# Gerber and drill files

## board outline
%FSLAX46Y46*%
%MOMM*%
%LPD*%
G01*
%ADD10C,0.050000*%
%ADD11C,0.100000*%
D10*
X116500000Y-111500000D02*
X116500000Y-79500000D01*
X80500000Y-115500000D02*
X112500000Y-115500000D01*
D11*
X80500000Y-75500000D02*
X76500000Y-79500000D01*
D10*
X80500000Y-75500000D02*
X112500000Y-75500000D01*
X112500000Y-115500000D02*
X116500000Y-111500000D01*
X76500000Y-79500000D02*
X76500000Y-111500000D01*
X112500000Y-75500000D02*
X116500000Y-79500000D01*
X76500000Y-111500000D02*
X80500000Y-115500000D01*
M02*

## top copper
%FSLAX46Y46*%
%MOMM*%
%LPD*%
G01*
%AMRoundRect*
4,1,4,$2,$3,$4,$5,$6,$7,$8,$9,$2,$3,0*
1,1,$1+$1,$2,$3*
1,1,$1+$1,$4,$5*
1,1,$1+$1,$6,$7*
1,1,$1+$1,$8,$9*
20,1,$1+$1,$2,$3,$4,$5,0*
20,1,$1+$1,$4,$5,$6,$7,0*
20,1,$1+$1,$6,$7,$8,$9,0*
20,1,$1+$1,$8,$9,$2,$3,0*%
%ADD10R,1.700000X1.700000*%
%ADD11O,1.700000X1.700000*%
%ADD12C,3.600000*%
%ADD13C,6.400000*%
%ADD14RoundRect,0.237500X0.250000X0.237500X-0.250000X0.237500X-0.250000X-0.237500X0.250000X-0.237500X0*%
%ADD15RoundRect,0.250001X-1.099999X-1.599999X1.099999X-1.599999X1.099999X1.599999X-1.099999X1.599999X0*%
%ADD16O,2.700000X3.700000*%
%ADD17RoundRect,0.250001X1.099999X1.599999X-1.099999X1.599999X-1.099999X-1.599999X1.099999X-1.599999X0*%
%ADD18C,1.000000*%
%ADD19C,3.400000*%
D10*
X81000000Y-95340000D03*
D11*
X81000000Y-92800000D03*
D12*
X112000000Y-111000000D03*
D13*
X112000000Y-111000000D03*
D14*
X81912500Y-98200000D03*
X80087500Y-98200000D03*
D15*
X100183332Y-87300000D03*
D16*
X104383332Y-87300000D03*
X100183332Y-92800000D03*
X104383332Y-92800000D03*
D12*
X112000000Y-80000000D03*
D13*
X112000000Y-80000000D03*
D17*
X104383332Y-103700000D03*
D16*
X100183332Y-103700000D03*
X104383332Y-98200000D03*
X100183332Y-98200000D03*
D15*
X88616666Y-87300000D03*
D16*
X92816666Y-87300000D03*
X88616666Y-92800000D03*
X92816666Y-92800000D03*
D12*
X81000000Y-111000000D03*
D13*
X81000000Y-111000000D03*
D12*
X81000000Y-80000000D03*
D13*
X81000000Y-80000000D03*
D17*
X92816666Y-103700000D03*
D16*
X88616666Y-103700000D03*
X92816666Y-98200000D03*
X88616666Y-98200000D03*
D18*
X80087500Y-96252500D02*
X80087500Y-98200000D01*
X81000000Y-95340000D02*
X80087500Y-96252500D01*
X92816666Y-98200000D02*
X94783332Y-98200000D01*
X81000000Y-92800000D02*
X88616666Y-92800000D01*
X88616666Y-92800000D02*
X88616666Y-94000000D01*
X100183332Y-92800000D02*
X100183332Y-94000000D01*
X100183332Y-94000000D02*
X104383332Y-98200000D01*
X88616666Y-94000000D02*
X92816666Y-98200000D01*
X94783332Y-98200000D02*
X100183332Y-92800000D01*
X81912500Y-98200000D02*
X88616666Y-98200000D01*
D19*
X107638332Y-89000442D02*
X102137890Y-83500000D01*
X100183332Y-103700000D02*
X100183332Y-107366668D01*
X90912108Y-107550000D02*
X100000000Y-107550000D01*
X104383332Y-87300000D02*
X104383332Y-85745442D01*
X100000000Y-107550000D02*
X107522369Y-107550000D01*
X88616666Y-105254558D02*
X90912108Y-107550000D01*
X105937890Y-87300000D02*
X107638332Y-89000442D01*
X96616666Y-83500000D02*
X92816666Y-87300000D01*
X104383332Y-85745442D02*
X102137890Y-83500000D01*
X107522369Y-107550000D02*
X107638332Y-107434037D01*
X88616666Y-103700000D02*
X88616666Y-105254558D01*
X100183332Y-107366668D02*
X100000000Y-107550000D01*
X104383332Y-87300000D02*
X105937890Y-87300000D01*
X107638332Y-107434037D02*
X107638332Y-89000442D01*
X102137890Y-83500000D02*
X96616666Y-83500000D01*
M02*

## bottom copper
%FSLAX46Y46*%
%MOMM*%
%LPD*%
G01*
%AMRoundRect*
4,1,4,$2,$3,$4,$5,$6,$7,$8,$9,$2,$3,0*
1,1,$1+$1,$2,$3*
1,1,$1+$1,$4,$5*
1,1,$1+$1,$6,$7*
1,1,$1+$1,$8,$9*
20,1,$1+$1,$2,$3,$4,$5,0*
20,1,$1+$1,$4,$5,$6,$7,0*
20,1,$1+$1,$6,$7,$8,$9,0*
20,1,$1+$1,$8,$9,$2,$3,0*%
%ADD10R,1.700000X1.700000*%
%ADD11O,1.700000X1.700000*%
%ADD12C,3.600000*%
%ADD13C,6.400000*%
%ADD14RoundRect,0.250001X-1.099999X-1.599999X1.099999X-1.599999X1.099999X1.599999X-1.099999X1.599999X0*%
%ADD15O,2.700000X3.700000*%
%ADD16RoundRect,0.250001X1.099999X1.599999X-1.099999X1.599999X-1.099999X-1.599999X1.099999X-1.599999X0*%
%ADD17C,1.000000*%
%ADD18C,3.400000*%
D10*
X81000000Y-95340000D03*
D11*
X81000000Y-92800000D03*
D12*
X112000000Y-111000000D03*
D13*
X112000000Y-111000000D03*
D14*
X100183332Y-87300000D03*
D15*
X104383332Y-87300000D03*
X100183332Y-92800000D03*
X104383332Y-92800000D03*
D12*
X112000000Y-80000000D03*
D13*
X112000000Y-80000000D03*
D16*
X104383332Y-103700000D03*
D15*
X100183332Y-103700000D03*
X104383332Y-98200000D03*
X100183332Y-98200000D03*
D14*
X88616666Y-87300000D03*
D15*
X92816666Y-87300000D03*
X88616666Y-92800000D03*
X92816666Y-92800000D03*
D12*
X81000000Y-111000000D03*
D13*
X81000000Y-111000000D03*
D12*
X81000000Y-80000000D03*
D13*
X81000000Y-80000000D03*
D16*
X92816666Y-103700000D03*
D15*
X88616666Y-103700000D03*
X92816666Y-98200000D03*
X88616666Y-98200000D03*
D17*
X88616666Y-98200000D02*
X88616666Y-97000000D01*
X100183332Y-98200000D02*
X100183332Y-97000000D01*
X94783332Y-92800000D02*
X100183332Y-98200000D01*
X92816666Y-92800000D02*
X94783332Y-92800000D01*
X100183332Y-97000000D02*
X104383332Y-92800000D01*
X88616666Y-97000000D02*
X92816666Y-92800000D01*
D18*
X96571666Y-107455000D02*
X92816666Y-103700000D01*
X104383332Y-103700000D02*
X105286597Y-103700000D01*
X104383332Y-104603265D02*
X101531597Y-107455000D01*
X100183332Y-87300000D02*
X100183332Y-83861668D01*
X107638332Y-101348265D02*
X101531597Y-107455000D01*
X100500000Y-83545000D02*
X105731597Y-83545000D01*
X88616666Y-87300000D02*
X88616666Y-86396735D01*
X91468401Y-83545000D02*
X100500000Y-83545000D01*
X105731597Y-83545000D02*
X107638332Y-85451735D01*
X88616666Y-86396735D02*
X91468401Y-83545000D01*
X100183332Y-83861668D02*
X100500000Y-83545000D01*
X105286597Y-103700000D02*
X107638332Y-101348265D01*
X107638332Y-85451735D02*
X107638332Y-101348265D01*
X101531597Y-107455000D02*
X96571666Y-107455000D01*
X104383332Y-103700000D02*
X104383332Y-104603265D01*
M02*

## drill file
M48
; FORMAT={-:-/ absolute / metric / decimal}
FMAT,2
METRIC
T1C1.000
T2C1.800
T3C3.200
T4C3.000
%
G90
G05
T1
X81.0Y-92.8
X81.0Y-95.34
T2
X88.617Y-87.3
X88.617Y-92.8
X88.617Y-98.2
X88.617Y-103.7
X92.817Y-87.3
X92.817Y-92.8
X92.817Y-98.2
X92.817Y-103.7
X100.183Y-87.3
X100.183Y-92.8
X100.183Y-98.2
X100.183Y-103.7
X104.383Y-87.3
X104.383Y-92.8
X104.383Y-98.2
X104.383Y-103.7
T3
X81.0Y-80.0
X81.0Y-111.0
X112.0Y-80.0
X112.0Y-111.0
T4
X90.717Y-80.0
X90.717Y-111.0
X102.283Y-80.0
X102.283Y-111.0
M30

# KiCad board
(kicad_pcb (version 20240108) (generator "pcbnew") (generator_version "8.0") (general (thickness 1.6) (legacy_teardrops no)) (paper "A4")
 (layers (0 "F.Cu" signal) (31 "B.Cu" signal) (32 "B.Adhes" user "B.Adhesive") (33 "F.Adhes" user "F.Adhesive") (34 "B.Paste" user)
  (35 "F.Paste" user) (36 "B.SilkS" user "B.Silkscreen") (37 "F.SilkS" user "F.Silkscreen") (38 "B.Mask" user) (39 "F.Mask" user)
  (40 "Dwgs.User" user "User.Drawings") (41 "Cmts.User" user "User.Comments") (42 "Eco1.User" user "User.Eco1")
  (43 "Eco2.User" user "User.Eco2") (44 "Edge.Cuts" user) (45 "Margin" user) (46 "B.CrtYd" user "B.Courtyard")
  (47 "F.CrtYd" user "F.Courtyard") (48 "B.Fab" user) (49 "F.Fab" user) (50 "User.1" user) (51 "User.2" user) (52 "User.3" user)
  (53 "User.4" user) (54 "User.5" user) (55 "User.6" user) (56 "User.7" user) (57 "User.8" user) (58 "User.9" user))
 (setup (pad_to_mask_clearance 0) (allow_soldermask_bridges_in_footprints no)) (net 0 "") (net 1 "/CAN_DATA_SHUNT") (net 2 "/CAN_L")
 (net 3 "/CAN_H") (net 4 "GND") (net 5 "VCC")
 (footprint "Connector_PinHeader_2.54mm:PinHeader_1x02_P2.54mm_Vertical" (layer "F.Cu") (at 81 95.34 180)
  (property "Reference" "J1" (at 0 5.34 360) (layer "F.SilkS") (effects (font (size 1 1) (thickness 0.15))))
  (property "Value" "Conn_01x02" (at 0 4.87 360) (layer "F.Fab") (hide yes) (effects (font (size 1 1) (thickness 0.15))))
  (pad "1" thru_hole rect (at 0 0 180) (size 1.7 1.7) (drill 1) (layers "*.Cu" "*.Mask") (remove_unused_layers no) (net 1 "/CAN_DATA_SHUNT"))
  (pad "2" thru_hole oval (at 0 2.54 180) (size 1.7 1.7) (drill 1) (layers "*.Cu" "*.Mask") (remove_unused_layers no) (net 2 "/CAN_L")))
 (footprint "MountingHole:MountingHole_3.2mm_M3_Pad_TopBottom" (layer "F.Cu") (at 112 111)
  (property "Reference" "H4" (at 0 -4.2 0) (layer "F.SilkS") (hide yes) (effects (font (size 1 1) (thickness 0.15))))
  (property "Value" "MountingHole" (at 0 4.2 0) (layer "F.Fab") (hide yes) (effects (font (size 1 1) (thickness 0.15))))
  (pad "1" thru_hole circle (at 0 0) (size 3.6 3.6) (drill 3.2) (layers "*.Cu" "*.Mask") (remove_unused_layers no))
  (pad "1" connect circle (at 0 0) (size 6.4 6.4) (layers "F.Cu" "F.Mask"))
  (pad "1" connect circle (at 0 0) (size 6.4 6.4) (layers "B.Cu" "B.Mask")))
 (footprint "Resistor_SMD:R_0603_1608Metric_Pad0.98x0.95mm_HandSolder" (layer "F.Cu") (at 81 98.2 180)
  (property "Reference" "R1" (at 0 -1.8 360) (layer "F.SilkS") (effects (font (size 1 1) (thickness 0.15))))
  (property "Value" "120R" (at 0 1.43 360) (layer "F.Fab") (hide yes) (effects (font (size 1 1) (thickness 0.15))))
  (pad "1" smd roundrect (at -0.9125 0 180) (size 0.975 0.95) (layers "F.Cu" "F.Paste" "F.Mask") (roundrect_rratio 0.25) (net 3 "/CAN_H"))
  (pad "2" smd roundrect (at 0.9125 0 180) (size 0.975 0.95) (layers "F.Cu" "F.Paste" "F.Mask") (roundrect_rratio 0.25)
   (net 1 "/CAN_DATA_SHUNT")))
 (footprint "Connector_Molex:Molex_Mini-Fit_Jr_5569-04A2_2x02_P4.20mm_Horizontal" (layer "F.Cu") (at 100.183332 87.3)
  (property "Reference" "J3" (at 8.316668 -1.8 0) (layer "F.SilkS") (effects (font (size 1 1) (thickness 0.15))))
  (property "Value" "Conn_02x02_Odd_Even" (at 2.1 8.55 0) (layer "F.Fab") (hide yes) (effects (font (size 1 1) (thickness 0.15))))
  (pad "" np_thru_hole circle (at 2.1 -7.3) (size 3 3) (drill 3) (layers "*.Cu" "*.Mask"))
  (pad "1" thru_hole roundrect (at 0 0) (size 2.7 3.7) (drill 1.8) (layers "*.Cu" "*.Mask") (remove_unused_layers no)
   (roundrect_rratio 0.092593) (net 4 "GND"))
  (pad "2" thru_hole oval (at 4.2 0) (size 2.7 3.7) (drill 1.8) (layers "*.Cu" "*.Mask") (remove_unused_layers no) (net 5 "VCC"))
  (pad "3" thru_hole oval (at 0 5.5) (size 2.7 3.7) (drill 1.8) (layers "*.Cu" "*.Mask") (remove_unused_layers no) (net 2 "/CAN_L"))
  (pad "4" thru_hole oval (at 4.2 5.5) (size 2.7 3.7) (drill 1.8) (layers "*.Cu" "*.Mask") (remove_unused_layers no) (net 3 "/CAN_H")))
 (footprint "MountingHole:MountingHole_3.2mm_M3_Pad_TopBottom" (layer "F.Cu") (at 112 80)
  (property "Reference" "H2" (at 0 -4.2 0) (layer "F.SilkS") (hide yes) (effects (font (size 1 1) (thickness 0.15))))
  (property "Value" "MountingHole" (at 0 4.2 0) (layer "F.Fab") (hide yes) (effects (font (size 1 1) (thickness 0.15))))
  (pad "1" thru_hole circle (at 0 0) (size 3.6 3.6) (drill 3.2) (layers "*.Cu" "*.Mask") (remove_unused_layers no))
  (pad "1" connect circle (at 0 0) (size 6.4 6.4) (layers "F.Cu" "F.Mask"))
  (pad "1" connect circle (at 0 0) (size 6.4 6.4) (layers "B.Cu" "B.Mask")))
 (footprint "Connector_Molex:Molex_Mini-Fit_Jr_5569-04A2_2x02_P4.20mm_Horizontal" (layer "F.Cu") (at 104.383332 103.7 180)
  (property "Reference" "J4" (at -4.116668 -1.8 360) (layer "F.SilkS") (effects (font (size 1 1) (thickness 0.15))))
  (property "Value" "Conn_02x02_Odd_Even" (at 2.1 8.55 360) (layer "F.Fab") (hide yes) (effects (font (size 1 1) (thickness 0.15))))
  (pad "" np_thru_hole circle (at 2.1 -7.3 180) (size 3 3) (drill 3) (layers "*.Cu" "*.Mask"))
  (pad "1" thru_hole roundrect (at 0 0 180) (size 2.7 3.7) (drill 1.8) (layers "*.Cu" "*.Mask") (remove_unused_layers no)
   (roundrect_rratio 0.092593) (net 4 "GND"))
  (pad "2" thru_hole oval (at 4.2 0 180) (size 2.7 3.7) (drill 1.8) (layers "*.Cu" "*.Mask") (remove_unused_layers no) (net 5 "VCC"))
  (pad "3" thru_hole oval (at 0 5.5 180) (size 2.7 3.7) (drill 1.8) (layers "*.Cu" "*.Mask") (remove_unused_layers no) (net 2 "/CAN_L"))
  (pad "4" thru_hole oval (at 4.2 5.5 180) (size 2.7 3.7) (drill 1.8) (layers "*.Cu" "*.Mask") (remove_unused_layers no) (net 3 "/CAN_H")))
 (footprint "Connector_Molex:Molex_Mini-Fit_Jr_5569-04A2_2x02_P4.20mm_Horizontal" (layer "F.Cu") (at 88.616666 87.3)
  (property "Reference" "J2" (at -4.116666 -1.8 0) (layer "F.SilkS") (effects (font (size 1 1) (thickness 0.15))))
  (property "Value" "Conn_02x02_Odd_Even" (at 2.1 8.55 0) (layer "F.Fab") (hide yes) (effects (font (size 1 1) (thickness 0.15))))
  (pad "" np_thru_hole circle (at 2.1 -7.3) (size 3 3) (drill 3) (layers "*.Cu" "*.Mask"))
  (pad "1" thru_hole roundrect (at 0 0) (size 2.7 3.7) (drill 1.8) (layers "*.Cu" "*.Mask") (remove_unused_layers no)
   (roundrect_rratio 0.092593) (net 4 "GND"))
  (pad "2" thru_hole oval (at 4.2 0) (size 2.7 3.7) (drill 1.8) (layers "*.Cu" "*.Mask") (remove_unused_layers no) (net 5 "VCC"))
  (pad "3" thru_hole oval (at 0 5.5) (size 2.7 3.7) (drill 1.8) (layers "*.Cu" "*.Mask") (remove_unused_layers no) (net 2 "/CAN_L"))
  (pad "4" thru_hole oval (at 4.2 5.5) (size 2.7 3.7) (drill 1.8) (layers "*.Cu" "*.Mask") (remove_unused_layers no) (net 3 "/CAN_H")))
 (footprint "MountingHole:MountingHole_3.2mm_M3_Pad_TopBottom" (layer "F.Cu") (at 81 111)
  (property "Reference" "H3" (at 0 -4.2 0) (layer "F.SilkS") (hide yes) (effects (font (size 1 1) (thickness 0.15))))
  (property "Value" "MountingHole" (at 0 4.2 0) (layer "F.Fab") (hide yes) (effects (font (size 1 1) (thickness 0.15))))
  (pad "1" thru_hole circle (at 0 0) (size 3.6 3.6) (drill 3.2) (layers "*.Cu" "*.Mask") (remove_unused_layers no))
  (pad "1" connect circle (at 0 0) (size 6.4 6.4) (layers "F.Cu" "F.Mask"))
  (pad "1" connect circle (at 0 0) (size 6.4 6.4) (layers "B.Cu" "B.Mask")))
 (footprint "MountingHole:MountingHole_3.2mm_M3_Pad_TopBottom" (layer "F.Cu") (at 81 80)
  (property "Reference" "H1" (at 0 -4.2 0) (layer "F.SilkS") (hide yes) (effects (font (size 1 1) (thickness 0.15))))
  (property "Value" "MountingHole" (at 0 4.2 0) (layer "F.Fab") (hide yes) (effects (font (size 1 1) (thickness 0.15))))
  (pad "1" thru_hole circle (at 0 0) (size 3.6 3.6) (drill 3.2) (layers "*.Cu" "*.Mask") (remove_unused_layers no))
  (pad "1" connect circle (at 0 0) (size 6.4 6.4) (layers "F.Cu" "F.Mask"))
  (pad "1" connect circle (at 0 0) (size 6.4 6.4) (layers "B.Cu" "B.Mask")))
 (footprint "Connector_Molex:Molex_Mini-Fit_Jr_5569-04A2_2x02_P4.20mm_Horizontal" (layer "F.Cu") (at 92.816666 103.7 180)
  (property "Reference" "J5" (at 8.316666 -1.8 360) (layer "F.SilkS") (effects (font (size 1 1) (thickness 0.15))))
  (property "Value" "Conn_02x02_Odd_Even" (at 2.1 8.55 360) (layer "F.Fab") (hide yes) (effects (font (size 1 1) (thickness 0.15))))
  (pad "" np_thru_hole circle (at 2.1 -7.3 180) (size 3 3) (drill 3) (layers "*.Cu" "*.Mask"))
  (pad "1" thru_hole roundrect (at 0 0 180) (size 2.7 3.7) (drill 1.8) (layers "*.Cu" "*.Mask") (remove_unused_layers no)
   (roundrect_rratio 0.092593) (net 4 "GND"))
  (pad "2" thru_hole oval (at 4.2 0 180) (size 2.7 3.7) (drill 1.8) (layers "*.Cu" "*.Mask") (remove_unused_layers no) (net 5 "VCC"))
  (pad "3" thru_hole oval (at 0 5.5 180) (size 2.7 3.7) (drill 1.8) (layers "*.Cu" "*.Mask") (remove_unused_layers no) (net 2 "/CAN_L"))
  (pad "4" thru_hole oval (at 4.2 5.5 180) (size 2.7 3.7) (drill 1.8) (layers "*.Cu" "*.Mask") (remove_unused_layers no) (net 3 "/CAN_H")))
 (gr_line (start 116.5 111.5) (end 116.5 79.5) (stroke (width 0.05) (type default)) (layer "Edge.Cuts"))
 (gr_line (start 80.5 115.5) (end 112.5 115.5) (stroke (width 0.05) (type default)) (layer "Edge.Cuts"))
 (gr_line (start 80.5 75.5) (end 76.5 79.5) (stroke (width 0.1) (type default)) (layer "Edge.Cuts"))
 (gr_line (start 80.5 75.5) (end 112.5 75.5) (stroke (width 0.05) (type default)) (layer "Edge.Cuts"))
 (gr_line (start 112.5 115.5) (end 116.5 111.5) (stroke (width 0.05) (type default)) (layer "Edge.Cuts"))
 (gr_line (start 76.5 79.5) (end 76.5 111.5) (stroke (width 0.05) (type default)) (layer "Edge.Cuts"))
 (gr_line (start 112.5 75.5) (end 116.5 79.5) (stroke (width 0.05) (type default)) (layer "Edge.Cuts"))
 (gr_line (start 76.5 111.5) (end 80.5 115.5) (stroke (width 0.05) (type default)) (layer "Edge.Cuts"))
 (segment (start 80.0875 96.2525) (end 80.0875 98.2) (width 1) (layer "F.Cu") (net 1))
 (segment (start 81 95.34) (end 80.0875 96.2525) (width 1) (layer "F.Cu") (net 1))
 (segment (start 92.816666 98.2) (end 94.783332 98.2) (width 1) (layer "F.Cu") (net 2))
 (segment (start 81 92.8) (end 88.616666 92.8) (width 1) (layer "F.Cu") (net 2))
 (segment (start 88.616666 92.8) (end 88.616666 94) (width 1) (layer "F.Cu") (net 2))
 (segment (start 100.183332 92.8) (end 100.183332 94) (width 1) (layer "F.Cu") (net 2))
 (segment (start 100.183332 94) (end 104.383332 98.2) (width 1) (layer "F.Cu") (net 2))
 (segment (start 88.616666 94) (end 92.816666 98.2) (width 1) (layer "F.Cu") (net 2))
 (segment (start 94.783332 98.2) (end 100.183332 92.8) (width 1) (layer "F.Cu") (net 2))
 (segment (start 81.9125 98.2) (end 88.616666 98.2) (width 1) (layer "F.Cu") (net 3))
 (segment (start 88.616666 98.2) (end 88.616666 97) (width 1) (layer "B.Cu") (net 3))
 (segment (start 100.183332 98.2) (end 100.183332 97) (width 1) (layer "B.Cu") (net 3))
 (segment (start 94.783332 92.8) (end 100.183332 98.2) (width 1) (layer "B.Cu") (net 3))
 (segment (start 92.816666 92.8) (end 94.783332 92.8) (width 1) (layer "B.Cu") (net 3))
 (segment (start 100.183332 97) (end 104.383332 92.8) (width 1) (layer "B.Cu") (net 3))
 (segment (start 88.616666 97) (end 92.816666 92.8) (width 1) (layer "B.Cu") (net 3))
 (segment (start 96.571666 107.455) (end 92.816666 103.7) (width 3.4) (layer "B.Cu") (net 4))
 (segment (start 104.383332 103.7) (end 105.286597 103.7) (width 3.4) (layer "B.Cu") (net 4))
 (segment (start 104.383332 104.603265) (end 101.531597 107.455) (width 3.4) (layer "B.Cu") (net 4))
 (segment (start 100.183332 87.3) (end 100.183332 83.861668) (width 3.4) (layer "B.Cu") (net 4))
 (segment (start 107.638332 101.348265) (end 101.531597 107.455) (width 3.4) (layer "B.Cu") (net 4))
 (segment (start 100.5 83.545) (end 105.731597 83.545) (width 3.4) (layer "B.Cu") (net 4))
 (segment (start 88.616666 87.3) (end 88.616666 86.396735) (width 3.4) (layer "B.Cu") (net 4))
 (segment (start 91.468401 83.545) (end 100.5 83.545) (width 3.4) (layer "B.Cu") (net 4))
 (segment (start 105.731597 83.545) (end 107.638332 85.451735) (width 3.4) (layer "B.Cu") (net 4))
 (segment (start 88.616666 86.396735) (end 91.468401 83.545) (width 3.4) (layer "B.Cu") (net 4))
 (segment (start 100.183332 83.861668) (end 100.5 83.545) (width 3.4) (layer "B.Cu") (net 4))
 (segment (start 105.286597 103.7) (end 107.638332 101.348265) (width 3.4) (layer "B.Cu") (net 4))
 (segment (start 107.638332 85.451735) (end 107.638332 101.348265) (width 3.4) (layer "B.Cu") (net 4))
 (segment (start 101.531597 107.455) (end 96.571666 107.455) (width 3.4) (layer "B.Cu") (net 4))
 (segment (start 104.383332 103.7) (end 104.383332 104.603265) (width 3.4) (layer "B.Cu") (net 4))
 (segment (start 107.638332 89.000442) (end 102.13789 83.5) (width 3.4) (layer "F.Cu") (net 5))
 (segment (start 100.183332 103.7) (end 100.183332 107.366668) (width 3.4) (layer "F.Cu") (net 5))
 (segment (start 90.912108 107.55) (end 100 107.55) (width 3.4) (layer "F.Cu") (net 5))
 (segment (start 104.383332 87.3) (end 104.383332 85.745442) (width 3.4) (layer "F.Cu") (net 5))
 (segment (start 100 107.55) (end 107.522369 107.55) (width 3.4) (layer "F.Cu") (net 5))
 (segment (start 88.616666 105.254558) (end 90.912108 107.55) (width 3.4) (layer "F.Cu") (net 5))
 (segment (start 105.93789 87.3) (end 107.638332 89.000442) (width 3.4) (layer "F.Cu") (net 5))
 (segment (start 96.616666 83.5) (end 92.816666 87.3) (width 3.4) (layer "F.Cu") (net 5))
 (segment (start 104.383332 85.745442) (end 102.13789 83.5) (width 3.4) (layer "F.Cu") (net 5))
 (segment (start 107.522369 107.55) (end 107.638332 107.434037) (width 3.4) (layer "F.Cu") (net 5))
 (segment (start 88.616666 103.7) (end 88.616666 105.254558) (width 3.4) (layer "F.Cu") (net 5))
 (segment (start 100.183332 107.366668) (end 100 107.55) (width 3.4) (layer "F.Cu") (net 5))
 (segment (start 104.383332 87.3) (end 105.93789 87.3) (width 3.4) (layer "F.Cu") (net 5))
 (segment (start 107.638332 107.434037) (end 107.638332 89.000442) (width 3.4) (layer "F.Cu") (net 5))
 (segment (start 102.13789 83.5) (end 96.616666 83.5) (width 3.4) (layer "F.Cu") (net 5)))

